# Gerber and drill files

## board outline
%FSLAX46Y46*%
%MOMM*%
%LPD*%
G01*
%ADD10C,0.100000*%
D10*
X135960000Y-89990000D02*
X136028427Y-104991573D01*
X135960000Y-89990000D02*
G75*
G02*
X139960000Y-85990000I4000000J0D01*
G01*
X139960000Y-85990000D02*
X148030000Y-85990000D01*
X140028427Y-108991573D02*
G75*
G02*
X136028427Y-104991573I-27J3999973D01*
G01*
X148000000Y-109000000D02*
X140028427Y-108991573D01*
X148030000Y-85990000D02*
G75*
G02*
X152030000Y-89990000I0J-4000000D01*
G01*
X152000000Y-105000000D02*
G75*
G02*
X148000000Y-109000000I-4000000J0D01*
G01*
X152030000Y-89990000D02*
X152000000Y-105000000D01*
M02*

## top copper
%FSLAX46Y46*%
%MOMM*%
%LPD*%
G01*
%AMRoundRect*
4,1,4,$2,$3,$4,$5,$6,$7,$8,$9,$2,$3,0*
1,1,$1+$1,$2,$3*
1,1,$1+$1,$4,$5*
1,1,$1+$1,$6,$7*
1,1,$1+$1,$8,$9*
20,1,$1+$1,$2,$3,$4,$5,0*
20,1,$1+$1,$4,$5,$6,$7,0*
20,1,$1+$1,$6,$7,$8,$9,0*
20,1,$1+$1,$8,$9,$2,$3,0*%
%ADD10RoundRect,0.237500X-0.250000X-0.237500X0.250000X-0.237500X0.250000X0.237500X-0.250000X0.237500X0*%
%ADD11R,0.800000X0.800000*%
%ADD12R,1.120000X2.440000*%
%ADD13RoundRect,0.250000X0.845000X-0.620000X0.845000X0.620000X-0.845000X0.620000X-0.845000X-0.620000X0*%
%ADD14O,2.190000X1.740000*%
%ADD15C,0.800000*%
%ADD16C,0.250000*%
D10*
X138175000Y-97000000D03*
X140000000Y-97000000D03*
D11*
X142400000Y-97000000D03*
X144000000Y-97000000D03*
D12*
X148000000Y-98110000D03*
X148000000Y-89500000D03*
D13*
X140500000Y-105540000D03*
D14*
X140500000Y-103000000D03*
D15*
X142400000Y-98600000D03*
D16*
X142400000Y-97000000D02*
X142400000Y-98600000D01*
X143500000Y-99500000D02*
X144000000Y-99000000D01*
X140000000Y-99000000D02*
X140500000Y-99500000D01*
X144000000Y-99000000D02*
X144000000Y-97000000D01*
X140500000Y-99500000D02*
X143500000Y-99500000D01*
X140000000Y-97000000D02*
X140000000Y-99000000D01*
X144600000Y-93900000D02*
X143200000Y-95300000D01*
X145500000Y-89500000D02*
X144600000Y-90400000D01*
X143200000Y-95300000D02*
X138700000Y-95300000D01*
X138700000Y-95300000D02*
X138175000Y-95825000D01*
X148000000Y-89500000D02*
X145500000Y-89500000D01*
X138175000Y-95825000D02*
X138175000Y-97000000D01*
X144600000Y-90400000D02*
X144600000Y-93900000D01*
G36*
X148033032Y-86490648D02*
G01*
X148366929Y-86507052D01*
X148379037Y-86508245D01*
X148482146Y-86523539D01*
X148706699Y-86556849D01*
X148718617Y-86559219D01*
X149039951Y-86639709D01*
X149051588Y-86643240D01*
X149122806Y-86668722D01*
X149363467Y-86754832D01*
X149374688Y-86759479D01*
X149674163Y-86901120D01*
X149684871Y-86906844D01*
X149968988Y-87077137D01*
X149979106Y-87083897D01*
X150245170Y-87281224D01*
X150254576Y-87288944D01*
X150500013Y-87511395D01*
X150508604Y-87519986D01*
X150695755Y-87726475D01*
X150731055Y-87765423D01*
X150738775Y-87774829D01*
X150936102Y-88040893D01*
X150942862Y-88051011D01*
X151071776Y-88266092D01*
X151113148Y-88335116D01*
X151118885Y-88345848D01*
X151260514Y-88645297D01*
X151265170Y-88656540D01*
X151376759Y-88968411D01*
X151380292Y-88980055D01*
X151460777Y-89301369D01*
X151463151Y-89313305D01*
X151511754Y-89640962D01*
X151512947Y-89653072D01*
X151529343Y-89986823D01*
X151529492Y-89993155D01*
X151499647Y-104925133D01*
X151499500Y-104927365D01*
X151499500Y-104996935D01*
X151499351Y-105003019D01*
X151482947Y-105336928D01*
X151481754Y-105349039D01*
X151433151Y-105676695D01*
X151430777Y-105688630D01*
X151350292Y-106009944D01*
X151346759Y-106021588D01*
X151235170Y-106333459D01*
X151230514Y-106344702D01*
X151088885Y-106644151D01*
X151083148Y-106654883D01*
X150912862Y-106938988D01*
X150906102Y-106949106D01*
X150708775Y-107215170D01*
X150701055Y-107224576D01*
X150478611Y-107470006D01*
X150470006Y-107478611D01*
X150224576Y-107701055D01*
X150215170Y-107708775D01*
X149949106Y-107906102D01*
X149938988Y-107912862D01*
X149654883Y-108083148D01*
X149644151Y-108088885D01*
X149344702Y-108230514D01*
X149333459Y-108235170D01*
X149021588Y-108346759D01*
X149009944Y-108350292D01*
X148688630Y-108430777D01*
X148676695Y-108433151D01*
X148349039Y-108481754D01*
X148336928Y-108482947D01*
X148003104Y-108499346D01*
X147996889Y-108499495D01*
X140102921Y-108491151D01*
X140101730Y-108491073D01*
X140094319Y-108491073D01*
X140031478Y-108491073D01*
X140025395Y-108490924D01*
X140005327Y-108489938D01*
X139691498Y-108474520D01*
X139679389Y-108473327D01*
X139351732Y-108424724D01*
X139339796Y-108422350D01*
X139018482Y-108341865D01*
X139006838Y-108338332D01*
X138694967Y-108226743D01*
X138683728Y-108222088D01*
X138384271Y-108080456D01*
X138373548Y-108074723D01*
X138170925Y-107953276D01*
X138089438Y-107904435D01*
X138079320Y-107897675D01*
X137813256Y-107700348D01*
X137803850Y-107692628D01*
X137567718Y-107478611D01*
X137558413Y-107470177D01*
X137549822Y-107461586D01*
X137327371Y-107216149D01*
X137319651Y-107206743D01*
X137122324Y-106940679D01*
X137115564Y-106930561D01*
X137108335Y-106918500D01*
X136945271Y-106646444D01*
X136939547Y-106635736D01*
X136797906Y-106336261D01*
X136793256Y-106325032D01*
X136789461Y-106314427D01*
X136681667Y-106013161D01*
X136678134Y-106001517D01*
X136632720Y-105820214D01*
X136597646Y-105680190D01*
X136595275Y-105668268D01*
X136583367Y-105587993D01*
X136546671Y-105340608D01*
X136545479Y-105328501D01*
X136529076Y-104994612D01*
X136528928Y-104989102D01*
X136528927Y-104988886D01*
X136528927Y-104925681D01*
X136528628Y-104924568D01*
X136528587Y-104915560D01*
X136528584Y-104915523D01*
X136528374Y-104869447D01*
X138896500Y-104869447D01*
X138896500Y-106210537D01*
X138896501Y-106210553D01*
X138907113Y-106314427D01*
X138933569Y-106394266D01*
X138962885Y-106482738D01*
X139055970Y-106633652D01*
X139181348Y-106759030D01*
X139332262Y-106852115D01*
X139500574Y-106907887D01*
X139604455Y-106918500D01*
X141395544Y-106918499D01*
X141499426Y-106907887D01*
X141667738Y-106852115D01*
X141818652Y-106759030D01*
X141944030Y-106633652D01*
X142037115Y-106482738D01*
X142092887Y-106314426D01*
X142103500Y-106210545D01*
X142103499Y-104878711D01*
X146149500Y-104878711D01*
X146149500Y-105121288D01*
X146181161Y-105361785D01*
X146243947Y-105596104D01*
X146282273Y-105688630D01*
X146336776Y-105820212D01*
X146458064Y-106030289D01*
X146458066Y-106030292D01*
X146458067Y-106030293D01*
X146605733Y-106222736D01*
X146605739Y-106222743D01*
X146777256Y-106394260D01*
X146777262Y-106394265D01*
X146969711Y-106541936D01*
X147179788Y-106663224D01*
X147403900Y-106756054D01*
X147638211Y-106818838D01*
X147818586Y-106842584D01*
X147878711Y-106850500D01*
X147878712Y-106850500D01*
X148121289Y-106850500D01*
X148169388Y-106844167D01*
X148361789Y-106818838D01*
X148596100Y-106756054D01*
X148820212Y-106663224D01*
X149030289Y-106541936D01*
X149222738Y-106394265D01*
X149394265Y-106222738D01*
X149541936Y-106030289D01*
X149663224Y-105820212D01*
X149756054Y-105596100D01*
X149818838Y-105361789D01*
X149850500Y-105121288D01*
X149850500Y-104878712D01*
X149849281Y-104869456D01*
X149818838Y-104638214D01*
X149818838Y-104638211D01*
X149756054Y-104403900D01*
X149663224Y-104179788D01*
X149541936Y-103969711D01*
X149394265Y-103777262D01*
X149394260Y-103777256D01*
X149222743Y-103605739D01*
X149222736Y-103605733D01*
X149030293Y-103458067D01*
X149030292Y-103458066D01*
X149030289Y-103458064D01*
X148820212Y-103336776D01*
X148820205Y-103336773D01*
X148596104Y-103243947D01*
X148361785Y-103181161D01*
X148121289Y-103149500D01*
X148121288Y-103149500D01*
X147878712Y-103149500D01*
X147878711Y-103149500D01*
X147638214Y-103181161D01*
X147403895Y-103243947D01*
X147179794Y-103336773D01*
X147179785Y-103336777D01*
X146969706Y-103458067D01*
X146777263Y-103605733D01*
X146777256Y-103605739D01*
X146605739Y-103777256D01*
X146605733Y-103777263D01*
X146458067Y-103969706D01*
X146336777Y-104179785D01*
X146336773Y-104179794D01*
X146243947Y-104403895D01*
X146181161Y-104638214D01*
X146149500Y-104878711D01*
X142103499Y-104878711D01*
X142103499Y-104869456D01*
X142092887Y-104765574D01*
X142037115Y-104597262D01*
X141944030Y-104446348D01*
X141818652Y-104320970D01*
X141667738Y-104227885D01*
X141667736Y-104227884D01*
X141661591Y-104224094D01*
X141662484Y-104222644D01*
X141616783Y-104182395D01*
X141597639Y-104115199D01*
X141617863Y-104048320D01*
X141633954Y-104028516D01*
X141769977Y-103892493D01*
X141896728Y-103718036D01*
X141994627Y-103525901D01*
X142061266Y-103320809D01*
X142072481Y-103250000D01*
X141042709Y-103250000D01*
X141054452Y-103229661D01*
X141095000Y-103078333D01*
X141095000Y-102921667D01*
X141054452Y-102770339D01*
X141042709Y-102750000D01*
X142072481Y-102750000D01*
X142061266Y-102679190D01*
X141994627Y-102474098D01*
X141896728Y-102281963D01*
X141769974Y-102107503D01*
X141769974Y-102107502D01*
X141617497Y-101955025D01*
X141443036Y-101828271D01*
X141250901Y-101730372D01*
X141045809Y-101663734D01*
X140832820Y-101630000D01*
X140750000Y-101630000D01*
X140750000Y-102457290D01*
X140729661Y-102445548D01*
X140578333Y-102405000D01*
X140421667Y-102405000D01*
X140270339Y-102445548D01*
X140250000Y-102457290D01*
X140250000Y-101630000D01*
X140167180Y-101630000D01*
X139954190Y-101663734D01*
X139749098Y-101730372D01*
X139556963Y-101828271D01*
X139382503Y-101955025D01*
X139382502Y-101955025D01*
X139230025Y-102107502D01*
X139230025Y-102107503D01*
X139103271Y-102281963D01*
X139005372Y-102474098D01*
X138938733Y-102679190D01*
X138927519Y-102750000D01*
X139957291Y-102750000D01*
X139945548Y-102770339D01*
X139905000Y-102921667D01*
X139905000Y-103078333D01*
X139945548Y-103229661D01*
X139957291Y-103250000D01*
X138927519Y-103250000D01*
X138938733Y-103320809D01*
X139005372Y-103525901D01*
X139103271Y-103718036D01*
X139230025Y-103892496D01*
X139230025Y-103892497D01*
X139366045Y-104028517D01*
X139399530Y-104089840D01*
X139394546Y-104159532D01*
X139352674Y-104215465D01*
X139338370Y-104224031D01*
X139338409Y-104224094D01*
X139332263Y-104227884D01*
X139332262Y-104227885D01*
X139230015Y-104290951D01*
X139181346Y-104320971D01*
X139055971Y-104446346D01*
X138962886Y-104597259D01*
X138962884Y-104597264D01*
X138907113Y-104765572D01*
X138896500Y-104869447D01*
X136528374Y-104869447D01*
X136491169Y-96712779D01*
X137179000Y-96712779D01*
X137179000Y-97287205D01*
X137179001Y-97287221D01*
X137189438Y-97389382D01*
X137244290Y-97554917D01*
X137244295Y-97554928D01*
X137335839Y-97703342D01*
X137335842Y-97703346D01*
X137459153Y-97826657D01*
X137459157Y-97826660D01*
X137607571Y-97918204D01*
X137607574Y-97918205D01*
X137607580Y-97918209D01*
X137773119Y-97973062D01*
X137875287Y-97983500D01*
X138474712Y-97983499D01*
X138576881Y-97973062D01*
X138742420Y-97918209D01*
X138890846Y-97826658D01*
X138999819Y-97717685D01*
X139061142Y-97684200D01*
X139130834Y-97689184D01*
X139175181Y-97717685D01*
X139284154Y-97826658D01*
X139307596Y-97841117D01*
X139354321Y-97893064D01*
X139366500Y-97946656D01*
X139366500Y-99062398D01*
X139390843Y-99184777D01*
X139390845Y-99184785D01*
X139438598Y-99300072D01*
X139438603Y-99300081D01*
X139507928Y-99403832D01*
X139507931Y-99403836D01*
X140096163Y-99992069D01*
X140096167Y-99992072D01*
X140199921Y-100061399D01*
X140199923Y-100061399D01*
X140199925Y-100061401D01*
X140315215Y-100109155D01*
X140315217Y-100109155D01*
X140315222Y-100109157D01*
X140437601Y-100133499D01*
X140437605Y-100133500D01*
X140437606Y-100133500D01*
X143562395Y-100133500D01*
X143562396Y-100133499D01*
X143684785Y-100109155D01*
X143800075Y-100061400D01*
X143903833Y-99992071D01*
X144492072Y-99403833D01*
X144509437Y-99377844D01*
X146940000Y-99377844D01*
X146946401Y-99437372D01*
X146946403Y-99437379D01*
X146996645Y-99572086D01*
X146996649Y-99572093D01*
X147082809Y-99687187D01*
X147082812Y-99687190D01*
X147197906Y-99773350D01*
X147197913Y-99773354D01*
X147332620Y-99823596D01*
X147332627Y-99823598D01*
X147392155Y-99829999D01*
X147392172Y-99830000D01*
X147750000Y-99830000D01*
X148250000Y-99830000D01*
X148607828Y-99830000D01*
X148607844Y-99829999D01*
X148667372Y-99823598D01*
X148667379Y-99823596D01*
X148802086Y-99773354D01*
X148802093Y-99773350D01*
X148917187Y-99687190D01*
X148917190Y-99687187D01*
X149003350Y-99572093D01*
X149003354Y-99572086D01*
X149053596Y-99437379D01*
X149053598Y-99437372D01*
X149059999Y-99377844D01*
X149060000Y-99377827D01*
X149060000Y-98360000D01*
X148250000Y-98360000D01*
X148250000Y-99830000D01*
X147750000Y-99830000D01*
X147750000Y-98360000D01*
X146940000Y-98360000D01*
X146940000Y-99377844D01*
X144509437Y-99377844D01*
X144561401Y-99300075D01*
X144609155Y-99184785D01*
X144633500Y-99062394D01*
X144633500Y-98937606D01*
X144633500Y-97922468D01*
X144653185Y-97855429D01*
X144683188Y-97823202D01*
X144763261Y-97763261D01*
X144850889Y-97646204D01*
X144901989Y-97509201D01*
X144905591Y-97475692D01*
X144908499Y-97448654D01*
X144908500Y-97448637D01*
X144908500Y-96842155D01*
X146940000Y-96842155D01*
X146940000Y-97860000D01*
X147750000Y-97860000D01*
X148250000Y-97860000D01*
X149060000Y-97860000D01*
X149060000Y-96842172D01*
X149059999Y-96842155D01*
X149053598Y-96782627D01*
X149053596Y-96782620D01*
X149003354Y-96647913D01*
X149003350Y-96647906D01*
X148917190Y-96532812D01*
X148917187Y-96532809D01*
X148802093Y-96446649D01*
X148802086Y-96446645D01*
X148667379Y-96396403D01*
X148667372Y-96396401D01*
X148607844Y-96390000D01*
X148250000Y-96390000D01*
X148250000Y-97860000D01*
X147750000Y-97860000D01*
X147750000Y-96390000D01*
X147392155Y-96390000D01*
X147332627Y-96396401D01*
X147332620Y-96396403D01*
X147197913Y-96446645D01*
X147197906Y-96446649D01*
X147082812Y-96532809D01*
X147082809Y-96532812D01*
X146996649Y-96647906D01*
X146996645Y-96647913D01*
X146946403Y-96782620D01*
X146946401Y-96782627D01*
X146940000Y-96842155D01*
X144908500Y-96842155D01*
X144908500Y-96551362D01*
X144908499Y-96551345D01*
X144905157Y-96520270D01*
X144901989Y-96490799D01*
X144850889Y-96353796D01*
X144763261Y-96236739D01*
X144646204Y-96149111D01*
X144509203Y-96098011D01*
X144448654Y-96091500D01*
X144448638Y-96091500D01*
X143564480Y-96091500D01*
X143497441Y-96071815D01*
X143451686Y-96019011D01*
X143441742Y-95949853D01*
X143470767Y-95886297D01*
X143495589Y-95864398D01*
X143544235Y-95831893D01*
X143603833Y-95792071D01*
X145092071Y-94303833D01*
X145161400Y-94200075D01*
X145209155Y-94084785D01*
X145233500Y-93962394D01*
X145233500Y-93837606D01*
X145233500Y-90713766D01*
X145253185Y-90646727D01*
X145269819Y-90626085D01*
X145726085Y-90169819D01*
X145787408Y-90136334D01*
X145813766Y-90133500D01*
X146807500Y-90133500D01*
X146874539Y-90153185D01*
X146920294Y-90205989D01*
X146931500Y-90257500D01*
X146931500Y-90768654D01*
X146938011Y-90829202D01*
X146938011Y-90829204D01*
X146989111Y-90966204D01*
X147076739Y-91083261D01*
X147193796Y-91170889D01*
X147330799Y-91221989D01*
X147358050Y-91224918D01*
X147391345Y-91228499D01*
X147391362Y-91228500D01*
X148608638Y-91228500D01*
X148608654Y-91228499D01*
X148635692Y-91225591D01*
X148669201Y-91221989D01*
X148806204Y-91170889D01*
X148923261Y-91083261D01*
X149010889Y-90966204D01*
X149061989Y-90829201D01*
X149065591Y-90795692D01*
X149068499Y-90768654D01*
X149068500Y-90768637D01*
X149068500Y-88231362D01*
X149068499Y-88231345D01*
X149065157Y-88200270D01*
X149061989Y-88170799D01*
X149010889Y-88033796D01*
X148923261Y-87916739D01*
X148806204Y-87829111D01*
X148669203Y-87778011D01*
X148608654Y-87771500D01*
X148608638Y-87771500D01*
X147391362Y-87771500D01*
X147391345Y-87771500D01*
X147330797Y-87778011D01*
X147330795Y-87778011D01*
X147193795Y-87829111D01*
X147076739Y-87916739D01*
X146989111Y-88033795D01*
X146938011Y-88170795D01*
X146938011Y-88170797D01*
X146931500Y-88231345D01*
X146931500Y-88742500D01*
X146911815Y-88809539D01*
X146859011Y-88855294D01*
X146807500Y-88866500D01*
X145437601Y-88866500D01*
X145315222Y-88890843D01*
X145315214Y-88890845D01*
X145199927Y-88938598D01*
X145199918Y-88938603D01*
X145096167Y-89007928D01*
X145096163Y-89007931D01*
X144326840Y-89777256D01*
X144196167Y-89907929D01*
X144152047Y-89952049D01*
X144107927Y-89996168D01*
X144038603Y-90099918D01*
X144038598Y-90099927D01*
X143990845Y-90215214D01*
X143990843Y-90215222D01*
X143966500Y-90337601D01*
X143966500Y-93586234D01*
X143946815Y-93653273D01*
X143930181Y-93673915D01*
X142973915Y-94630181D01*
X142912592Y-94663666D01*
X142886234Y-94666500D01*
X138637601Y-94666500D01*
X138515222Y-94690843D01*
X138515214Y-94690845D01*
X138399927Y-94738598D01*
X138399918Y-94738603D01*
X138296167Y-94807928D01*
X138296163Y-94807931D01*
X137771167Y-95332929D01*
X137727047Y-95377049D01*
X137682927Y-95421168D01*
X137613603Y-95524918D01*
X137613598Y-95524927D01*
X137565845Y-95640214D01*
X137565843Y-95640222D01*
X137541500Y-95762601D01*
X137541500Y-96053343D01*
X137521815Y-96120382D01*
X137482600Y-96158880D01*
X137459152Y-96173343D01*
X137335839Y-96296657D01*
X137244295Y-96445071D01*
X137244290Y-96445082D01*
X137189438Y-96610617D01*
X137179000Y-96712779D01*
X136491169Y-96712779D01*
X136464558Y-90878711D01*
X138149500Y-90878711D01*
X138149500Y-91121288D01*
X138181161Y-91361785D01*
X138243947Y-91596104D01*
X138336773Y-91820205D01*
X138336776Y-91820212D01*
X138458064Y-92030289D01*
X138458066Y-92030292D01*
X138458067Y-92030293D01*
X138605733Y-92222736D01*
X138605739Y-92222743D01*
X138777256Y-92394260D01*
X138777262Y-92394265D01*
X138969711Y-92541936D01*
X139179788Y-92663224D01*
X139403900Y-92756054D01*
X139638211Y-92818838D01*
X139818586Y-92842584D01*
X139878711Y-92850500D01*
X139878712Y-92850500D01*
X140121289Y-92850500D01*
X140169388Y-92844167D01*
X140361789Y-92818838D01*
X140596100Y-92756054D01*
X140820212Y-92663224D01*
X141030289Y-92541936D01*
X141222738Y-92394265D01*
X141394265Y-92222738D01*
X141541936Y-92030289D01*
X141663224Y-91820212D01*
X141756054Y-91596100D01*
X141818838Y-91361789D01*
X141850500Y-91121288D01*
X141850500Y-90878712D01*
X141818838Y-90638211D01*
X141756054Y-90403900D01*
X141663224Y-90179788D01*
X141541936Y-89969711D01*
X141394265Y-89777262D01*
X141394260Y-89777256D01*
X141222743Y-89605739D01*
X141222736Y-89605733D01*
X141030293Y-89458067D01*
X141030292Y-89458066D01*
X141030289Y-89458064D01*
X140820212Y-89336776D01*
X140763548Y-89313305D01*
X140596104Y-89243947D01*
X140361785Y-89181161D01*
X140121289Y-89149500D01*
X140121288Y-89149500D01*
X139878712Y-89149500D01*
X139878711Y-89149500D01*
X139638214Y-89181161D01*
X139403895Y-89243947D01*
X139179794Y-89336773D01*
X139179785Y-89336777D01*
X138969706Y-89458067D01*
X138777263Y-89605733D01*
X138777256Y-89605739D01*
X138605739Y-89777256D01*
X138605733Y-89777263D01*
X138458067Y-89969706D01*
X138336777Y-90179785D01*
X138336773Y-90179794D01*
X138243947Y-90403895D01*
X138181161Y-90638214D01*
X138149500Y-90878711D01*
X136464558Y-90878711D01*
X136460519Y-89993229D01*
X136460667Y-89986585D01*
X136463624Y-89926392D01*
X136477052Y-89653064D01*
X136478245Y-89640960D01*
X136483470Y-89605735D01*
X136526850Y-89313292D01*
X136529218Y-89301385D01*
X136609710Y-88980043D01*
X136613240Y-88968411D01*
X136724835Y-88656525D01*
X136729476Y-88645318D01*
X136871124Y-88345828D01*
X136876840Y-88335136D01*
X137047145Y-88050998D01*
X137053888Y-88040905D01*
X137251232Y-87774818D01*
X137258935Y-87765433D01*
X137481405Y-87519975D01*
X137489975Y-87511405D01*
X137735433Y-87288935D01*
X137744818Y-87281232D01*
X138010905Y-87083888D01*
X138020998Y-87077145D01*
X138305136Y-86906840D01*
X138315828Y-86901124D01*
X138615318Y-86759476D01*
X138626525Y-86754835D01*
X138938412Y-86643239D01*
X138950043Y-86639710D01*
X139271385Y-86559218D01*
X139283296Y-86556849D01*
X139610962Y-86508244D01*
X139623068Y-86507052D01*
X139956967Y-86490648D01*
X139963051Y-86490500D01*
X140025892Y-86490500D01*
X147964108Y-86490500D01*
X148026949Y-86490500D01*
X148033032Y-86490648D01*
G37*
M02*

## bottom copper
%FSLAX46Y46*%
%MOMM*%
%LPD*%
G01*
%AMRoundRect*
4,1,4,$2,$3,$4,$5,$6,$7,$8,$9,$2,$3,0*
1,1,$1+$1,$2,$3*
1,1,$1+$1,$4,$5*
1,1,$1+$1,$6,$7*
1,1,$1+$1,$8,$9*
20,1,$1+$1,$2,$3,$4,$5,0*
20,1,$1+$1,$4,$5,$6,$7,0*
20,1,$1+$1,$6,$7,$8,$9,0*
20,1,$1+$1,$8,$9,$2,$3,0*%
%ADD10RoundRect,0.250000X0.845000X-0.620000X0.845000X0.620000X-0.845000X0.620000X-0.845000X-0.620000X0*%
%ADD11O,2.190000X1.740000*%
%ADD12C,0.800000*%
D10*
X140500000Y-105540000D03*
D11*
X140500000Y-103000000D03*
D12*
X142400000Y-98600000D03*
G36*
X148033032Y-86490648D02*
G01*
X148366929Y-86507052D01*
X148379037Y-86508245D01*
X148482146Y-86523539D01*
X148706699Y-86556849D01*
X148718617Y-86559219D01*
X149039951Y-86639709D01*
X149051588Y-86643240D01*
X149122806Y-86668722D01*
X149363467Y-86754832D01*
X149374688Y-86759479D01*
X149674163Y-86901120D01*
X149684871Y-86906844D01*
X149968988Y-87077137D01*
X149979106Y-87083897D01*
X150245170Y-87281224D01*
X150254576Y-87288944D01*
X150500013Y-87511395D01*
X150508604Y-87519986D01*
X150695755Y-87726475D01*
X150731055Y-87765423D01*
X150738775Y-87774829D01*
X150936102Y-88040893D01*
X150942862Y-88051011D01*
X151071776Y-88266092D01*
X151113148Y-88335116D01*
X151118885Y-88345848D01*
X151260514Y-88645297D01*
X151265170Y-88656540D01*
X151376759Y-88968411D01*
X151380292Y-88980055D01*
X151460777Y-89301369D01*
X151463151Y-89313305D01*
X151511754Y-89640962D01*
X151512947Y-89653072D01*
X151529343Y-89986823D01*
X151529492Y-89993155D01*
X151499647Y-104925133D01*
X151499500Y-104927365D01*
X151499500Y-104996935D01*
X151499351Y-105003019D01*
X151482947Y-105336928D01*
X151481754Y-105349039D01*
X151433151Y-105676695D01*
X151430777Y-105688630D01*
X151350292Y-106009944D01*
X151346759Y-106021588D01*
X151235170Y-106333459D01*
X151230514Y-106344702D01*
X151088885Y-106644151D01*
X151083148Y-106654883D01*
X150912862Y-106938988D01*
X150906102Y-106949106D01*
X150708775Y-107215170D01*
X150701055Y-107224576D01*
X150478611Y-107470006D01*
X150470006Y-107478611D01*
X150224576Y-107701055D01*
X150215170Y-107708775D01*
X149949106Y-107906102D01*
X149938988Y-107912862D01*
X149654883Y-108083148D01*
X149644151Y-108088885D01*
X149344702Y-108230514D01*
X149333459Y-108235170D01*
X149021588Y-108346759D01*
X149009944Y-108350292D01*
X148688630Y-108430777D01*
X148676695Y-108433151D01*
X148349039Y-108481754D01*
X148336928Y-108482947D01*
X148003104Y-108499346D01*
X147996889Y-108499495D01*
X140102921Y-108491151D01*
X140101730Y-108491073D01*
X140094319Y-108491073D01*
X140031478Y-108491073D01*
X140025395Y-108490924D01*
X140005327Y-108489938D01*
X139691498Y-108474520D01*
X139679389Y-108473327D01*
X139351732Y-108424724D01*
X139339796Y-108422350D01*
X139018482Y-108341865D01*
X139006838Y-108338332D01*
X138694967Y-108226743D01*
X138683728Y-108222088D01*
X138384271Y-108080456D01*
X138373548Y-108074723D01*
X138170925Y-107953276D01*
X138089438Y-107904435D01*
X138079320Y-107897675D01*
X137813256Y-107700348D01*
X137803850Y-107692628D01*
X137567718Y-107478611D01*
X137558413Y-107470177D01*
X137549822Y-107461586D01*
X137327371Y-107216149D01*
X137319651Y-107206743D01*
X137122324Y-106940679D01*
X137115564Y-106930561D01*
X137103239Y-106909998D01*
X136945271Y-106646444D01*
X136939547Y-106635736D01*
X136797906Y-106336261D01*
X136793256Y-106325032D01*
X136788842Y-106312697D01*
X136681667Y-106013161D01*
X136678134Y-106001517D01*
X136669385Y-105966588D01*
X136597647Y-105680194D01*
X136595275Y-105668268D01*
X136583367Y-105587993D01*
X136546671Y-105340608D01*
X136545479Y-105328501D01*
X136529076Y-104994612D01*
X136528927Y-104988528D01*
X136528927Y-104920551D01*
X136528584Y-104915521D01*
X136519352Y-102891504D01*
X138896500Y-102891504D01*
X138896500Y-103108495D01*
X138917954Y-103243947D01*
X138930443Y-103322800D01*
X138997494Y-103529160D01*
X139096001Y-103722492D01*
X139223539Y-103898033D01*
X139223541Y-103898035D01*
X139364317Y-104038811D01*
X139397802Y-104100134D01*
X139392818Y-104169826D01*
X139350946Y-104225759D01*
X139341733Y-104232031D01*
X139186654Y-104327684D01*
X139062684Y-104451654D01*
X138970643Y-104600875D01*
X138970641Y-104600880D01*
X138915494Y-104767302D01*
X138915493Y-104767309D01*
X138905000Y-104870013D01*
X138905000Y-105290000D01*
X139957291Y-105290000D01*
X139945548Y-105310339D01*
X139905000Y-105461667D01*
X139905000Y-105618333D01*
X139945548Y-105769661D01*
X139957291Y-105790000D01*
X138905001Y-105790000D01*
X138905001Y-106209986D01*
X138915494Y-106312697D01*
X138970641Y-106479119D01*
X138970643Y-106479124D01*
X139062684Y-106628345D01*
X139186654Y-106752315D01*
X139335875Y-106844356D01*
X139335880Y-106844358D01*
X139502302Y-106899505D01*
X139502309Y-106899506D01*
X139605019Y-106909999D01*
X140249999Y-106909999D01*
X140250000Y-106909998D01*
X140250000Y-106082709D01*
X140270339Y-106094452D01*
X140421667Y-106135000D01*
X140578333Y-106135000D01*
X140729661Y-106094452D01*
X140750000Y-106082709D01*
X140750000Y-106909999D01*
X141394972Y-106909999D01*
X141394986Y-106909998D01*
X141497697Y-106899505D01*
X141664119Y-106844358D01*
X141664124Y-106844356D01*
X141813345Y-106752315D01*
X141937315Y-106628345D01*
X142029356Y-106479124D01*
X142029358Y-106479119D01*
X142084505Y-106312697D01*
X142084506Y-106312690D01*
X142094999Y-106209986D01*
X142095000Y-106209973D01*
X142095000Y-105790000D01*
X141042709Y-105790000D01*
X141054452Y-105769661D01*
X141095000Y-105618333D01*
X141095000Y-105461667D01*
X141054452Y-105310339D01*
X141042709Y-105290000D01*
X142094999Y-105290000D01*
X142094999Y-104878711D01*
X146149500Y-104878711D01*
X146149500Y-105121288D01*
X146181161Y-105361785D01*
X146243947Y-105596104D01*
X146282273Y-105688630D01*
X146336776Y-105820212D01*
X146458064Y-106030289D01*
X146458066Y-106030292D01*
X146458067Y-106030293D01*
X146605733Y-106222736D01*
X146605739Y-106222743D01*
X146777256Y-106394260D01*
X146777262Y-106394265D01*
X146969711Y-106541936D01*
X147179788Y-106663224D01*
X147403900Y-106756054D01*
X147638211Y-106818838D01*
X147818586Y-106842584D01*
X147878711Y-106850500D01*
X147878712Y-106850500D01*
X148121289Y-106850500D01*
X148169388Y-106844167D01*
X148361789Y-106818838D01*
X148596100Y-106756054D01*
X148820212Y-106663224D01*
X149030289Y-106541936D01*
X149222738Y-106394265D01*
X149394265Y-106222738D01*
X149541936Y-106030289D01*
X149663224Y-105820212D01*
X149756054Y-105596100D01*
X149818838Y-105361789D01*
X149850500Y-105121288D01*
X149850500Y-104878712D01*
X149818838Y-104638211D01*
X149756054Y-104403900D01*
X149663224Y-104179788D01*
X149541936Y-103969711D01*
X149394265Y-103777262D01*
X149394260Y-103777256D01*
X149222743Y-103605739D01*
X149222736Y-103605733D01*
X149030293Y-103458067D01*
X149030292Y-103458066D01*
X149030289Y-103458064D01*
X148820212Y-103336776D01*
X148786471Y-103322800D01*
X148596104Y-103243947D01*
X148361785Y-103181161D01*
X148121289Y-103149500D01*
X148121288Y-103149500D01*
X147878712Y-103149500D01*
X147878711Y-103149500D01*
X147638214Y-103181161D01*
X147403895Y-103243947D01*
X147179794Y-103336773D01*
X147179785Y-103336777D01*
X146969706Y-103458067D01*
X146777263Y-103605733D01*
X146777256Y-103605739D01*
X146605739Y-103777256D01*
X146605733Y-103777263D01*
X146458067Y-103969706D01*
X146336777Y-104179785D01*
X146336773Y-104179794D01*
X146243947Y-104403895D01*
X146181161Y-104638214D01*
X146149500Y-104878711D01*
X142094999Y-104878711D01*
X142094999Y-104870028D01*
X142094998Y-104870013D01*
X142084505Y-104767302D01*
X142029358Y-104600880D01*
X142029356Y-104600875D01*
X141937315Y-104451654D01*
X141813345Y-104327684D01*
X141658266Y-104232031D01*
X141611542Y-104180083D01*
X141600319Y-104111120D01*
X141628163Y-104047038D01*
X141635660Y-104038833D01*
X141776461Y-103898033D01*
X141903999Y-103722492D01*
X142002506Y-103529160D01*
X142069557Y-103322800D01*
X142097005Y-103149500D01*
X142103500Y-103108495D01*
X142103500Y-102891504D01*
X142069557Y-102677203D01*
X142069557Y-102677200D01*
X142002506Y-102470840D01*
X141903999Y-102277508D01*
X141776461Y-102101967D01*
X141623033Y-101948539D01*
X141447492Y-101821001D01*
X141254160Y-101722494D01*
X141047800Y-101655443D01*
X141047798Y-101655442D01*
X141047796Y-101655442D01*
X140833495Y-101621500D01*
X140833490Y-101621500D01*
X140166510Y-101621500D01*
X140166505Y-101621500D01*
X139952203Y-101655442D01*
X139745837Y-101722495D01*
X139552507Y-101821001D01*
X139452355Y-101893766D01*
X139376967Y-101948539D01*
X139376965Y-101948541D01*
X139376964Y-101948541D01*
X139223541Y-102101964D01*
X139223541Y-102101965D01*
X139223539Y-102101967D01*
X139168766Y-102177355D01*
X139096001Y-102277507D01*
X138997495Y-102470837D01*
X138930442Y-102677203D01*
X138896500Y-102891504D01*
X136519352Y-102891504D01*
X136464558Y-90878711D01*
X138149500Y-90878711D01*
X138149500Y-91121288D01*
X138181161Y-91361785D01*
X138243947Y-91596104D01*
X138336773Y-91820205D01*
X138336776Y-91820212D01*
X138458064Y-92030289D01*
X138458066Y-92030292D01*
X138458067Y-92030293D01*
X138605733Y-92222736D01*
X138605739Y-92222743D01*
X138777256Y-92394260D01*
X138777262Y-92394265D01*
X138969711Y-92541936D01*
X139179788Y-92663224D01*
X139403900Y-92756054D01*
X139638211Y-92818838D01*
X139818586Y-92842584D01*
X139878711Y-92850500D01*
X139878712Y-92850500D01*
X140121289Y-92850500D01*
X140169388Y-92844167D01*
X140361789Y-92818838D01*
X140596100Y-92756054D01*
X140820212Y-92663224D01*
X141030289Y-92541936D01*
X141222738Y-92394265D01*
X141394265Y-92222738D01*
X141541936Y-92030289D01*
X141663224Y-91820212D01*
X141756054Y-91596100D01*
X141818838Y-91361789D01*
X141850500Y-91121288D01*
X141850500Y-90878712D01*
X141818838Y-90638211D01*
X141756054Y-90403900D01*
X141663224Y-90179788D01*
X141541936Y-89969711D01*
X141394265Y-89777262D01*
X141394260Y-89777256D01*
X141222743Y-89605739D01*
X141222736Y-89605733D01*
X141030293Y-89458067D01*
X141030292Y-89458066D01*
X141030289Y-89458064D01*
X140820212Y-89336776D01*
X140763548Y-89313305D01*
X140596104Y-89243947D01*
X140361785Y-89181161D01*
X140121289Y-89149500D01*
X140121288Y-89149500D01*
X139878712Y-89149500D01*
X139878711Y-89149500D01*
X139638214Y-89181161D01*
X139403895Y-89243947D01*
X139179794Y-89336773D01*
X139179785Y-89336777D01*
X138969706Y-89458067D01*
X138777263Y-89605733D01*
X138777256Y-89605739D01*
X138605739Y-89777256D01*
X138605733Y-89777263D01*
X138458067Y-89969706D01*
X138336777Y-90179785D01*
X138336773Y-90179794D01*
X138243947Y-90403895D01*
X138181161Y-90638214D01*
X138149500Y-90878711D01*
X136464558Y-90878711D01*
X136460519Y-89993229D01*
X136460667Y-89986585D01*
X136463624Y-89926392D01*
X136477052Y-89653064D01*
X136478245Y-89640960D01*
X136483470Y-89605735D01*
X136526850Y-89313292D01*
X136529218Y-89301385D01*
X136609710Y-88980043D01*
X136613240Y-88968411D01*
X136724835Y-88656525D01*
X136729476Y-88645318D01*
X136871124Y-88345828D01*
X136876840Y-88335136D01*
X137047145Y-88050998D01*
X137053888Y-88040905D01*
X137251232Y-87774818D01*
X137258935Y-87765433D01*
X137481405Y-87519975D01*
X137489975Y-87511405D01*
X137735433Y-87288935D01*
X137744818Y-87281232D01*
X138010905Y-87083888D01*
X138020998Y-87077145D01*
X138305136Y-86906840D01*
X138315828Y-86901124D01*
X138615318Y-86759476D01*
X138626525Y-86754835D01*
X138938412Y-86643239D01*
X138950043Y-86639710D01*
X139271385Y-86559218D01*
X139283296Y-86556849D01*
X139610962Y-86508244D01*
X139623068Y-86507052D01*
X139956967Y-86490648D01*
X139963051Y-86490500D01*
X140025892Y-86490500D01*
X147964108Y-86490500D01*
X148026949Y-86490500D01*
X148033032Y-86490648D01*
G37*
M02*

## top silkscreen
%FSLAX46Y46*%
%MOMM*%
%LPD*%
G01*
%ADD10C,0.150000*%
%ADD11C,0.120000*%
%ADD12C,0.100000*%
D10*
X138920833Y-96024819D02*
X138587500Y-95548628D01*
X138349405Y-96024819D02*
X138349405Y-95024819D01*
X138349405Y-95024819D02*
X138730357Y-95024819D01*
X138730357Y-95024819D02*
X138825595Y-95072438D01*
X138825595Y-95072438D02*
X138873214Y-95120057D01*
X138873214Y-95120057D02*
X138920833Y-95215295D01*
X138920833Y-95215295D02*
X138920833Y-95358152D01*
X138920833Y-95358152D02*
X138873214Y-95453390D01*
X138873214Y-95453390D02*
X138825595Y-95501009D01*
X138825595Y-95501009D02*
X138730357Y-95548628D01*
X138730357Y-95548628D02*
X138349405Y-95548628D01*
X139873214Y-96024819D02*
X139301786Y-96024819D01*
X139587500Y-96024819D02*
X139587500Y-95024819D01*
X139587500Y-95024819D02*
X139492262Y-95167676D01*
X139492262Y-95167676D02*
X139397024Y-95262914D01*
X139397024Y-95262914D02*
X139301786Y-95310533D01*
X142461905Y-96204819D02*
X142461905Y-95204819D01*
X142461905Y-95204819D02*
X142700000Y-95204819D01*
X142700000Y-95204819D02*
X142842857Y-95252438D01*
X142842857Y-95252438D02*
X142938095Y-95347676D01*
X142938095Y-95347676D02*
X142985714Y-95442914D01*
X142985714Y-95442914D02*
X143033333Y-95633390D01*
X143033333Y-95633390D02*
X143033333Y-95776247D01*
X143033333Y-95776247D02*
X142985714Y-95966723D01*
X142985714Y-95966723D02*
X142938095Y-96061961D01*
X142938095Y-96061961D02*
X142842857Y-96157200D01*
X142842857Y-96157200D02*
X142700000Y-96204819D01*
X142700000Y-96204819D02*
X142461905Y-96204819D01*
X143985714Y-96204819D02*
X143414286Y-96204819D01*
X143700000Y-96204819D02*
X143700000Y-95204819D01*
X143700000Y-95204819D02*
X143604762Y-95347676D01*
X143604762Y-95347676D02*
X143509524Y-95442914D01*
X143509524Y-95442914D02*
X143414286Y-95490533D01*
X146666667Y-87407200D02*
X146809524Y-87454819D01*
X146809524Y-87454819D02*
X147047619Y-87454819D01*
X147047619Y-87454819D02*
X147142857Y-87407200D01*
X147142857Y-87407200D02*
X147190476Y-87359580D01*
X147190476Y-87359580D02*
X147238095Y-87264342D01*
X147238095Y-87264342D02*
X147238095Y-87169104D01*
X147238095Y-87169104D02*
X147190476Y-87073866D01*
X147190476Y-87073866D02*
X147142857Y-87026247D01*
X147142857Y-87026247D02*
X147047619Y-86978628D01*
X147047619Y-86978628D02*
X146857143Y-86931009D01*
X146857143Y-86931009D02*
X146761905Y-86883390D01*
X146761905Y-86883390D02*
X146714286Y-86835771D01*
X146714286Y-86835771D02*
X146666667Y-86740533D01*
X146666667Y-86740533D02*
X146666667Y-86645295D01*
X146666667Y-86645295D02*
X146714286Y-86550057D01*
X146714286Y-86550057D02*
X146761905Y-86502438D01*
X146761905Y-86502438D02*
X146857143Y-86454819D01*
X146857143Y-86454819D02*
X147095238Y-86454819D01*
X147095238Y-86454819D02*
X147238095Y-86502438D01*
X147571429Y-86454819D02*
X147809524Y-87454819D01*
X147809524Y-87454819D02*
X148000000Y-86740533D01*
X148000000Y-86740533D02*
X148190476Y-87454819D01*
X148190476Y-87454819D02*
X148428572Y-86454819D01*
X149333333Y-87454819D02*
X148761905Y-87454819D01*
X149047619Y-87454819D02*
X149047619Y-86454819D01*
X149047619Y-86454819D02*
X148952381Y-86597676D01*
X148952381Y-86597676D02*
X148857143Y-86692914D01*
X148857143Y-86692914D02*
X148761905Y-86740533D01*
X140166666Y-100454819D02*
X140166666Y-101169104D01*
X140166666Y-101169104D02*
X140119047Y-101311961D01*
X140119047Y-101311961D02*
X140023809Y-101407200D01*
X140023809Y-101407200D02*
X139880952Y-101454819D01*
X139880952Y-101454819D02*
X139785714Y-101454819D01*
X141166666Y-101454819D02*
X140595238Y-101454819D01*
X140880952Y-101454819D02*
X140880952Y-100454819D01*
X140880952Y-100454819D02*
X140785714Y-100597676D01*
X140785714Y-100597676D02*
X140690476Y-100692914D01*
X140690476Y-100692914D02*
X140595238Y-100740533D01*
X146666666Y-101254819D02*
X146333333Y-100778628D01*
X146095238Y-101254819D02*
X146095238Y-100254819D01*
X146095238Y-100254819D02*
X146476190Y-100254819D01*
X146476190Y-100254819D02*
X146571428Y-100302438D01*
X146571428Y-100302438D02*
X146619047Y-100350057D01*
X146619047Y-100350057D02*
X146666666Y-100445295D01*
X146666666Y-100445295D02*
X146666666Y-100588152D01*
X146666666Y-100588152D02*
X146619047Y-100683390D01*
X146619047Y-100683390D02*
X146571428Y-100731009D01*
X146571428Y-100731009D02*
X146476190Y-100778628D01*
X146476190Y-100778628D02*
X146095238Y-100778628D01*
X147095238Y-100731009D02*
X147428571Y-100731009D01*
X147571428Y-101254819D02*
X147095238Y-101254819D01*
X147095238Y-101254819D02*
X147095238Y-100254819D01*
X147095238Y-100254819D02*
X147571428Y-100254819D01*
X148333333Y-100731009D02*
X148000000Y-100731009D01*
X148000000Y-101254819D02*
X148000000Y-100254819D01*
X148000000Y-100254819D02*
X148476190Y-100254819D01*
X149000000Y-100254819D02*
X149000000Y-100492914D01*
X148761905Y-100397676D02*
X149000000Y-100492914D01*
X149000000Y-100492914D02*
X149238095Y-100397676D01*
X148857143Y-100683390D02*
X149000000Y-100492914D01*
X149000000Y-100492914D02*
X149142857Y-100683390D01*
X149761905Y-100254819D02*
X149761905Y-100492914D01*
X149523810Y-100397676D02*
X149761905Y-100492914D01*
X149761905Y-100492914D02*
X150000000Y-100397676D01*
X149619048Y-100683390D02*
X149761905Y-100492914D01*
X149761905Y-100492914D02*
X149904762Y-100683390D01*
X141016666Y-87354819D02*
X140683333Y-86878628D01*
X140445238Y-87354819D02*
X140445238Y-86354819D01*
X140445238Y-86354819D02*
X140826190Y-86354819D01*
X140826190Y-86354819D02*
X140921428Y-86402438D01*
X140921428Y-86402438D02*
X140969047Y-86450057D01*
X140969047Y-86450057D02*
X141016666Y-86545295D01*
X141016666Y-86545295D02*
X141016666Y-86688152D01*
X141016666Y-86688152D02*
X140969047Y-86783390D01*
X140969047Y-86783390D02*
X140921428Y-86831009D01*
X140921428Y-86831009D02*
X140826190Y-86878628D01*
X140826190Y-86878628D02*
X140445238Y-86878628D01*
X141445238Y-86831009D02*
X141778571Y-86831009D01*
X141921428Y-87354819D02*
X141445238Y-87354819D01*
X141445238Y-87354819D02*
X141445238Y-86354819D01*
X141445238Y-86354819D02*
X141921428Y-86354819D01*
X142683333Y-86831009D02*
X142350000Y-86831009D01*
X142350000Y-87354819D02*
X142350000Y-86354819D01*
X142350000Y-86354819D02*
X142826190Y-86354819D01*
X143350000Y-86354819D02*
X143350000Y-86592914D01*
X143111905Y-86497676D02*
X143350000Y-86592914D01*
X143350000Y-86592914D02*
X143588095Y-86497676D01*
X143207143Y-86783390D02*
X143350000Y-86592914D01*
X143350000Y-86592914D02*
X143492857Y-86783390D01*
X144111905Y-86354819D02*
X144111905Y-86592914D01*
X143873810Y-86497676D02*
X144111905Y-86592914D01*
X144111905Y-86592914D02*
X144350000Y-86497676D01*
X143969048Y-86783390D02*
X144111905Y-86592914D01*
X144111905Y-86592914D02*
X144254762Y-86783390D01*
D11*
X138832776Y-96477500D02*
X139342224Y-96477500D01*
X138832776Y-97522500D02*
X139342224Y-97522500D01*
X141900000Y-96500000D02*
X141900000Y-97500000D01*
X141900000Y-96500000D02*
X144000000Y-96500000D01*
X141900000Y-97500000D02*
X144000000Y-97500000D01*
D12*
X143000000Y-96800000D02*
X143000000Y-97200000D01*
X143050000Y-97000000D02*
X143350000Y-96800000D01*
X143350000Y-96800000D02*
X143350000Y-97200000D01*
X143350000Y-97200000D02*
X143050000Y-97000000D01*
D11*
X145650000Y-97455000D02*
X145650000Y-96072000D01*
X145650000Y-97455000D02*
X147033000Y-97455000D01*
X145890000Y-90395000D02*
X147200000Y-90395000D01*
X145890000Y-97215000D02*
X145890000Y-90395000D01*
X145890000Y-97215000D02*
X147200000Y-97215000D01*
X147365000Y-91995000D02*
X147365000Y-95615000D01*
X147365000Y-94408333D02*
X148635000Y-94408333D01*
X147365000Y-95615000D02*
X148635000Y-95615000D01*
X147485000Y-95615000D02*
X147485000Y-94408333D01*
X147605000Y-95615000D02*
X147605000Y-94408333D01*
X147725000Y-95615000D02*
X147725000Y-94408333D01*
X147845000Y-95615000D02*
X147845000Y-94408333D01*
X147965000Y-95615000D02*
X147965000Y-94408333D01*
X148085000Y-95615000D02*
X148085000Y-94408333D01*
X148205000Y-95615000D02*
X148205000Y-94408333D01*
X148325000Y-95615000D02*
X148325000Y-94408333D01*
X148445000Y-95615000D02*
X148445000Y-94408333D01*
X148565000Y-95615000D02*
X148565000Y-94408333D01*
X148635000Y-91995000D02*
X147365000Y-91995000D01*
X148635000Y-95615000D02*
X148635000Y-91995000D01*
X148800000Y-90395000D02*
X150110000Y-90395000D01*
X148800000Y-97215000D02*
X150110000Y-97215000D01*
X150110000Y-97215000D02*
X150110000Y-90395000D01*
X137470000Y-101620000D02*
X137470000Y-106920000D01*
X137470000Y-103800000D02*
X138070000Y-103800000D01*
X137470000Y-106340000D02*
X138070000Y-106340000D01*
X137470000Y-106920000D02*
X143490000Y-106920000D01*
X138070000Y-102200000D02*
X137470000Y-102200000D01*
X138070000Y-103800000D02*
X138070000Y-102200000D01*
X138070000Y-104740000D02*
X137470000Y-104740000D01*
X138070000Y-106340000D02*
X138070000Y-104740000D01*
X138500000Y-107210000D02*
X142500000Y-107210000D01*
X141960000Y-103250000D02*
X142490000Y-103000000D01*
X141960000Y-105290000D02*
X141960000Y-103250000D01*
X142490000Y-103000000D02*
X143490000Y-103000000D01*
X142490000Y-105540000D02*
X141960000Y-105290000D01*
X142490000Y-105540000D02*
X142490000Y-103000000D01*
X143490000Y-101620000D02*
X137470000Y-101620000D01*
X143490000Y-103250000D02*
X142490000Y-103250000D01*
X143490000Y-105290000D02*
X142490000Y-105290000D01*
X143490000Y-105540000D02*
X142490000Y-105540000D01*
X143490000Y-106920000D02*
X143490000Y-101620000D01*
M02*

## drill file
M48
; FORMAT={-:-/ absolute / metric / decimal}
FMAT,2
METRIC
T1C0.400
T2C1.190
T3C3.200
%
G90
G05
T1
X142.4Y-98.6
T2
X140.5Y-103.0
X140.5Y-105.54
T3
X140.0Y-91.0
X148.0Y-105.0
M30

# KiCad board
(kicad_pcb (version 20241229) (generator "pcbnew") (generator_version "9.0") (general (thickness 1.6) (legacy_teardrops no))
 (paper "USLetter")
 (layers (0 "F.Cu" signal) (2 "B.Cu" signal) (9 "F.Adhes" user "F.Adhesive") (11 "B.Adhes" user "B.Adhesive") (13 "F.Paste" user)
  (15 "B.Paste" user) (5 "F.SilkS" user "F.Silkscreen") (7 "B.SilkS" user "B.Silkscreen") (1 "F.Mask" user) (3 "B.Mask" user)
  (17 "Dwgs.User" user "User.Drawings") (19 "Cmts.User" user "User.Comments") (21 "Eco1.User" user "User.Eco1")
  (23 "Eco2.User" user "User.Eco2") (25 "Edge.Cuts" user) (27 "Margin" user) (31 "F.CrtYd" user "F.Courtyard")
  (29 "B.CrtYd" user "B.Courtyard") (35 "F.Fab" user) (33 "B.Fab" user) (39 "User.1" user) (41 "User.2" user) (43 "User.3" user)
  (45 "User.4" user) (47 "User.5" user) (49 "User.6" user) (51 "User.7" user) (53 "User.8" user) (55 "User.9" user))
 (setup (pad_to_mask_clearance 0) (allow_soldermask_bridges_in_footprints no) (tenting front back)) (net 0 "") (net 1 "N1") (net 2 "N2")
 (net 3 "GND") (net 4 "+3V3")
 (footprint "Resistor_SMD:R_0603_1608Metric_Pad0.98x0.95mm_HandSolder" (layer "F.Cu") (at 139.0875 97)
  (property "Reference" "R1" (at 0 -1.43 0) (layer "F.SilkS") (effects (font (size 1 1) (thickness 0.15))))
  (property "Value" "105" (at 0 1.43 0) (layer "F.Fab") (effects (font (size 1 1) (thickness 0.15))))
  (fp_line (start -0.254724 -0.5225) (end 0.254724 -0.5225) (stroke (width 0.12) (type solid)) (layer "F.SilkS"))
  (fp_line (start -0.254724 0.5225) (end 0.254724 0.5225) (stroke (width 0.12) (type solid)) (layer "F.SilkS"))
  (pad "1" smd roundrect (at -0.9125 0) (size 0.975 0.95) (layers "F.Cu" "F.Mask" "F.Paste") (roundrect_rratio 0.25) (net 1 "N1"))
  (pad "2" smd roundrect (at 0.9125 0) (size 0.975 0.95) (layers "F.Cu" "F.Mask" "F.Paste") (roundrect_rratio 0.25) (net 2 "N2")))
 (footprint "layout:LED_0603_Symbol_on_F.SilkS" (layer "F.Cu") (at 143.2 97)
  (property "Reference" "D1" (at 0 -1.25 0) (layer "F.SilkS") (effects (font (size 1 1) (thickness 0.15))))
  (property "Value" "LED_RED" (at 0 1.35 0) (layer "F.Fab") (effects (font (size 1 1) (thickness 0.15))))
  (fp_line (start -1.3 -0.5) (end -1.3 0.5) (stroke (width 0.12) (type solid)) (layer "F.SilkS"))
  (fp_line (start -1.3 -0.5) (end 0.8 -0.5) (stroke (width 0.12) (type solid)) (layer "F.SilkS"))
  (fp_line (start -1.3 0.5) (end 0.8 0.5) (stroke (width 0.12) (type solid)) (layer "F.SilkS"))
  (fp_line (start -0.2 -0.2) (end -0.2 0.2) (stroke (width 0.1) (type solid)) (layer "F.SilkS"))
  (fp_line (start -0.15 0) (end 0.15 -0.2) (stroke (width 0.1) (type solid)) (layer "F.SilkS"))
  (fp_line (start 0.15 -0.2) (end 0.15 0.2) (stroke (width 0.1) (type solid)) (layer "F.SilkS"))
  (fp_line (start 0.15 0.2) (end -0.15 0) (stroke (width 0.1) (type solid)) (layer "F.SilkS"))
  (pad "1" smd rect (at -0.8 0 180) (size 0.8 0.8) (layers "F.Cu" "F.Mask" "F.Paste") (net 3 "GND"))
  (pad "2" smd rect (at 0.8 0 180) (size 0.8 0.8) (layers "F.Cu" "F.Mask" "F.Paste") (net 2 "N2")))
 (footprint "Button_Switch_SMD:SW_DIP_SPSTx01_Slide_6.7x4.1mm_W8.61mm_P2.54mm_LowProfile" (layer "F.Cu") (at 148 93.805 90)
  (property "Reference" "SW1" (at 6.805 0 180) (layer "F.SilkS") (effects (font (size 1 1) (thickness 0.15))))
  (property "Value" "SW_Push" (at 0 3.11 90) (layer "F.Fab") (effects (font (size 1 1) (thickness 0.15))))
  (fp_line (start -3.65 -2.35) (end -2.267 -2.35) (stroke (width 0.12) (type solid)) (layer "F.SilkS"))
  (fp_line (start -3.65 -2.35) (end -3.65 -0.967) (stroke (width 0.12) (type solid)) (layer "F.SilkS"))
  (fp_line (start 3.41 -2.11) (end 3.41 -0.8) (stroke (width 0.12) (type solid)) (layer "F.SilkS"))
  (fp_line (start -3.41 -2.11) (end 3.41 -2.11) (stroke (width 0.12) (type solid)) (layer "F.SilkS"))
  (fp_line (start -3.41 -2.11) (end -3.41 -0.8) (stroke (width 0.12) (type solid)) (layer "F.SilkS"))
  (fp_line (start 1.81 -0.635) (end -1.81 -0.635) (stroke (width 0.12) (type solid)) (layer "F.SilkS"))
  (fp_line (start -0.603333 -0.635) (end -0.603333 0.635) (stroke (width 0.12) (type solid)) (layer "F.SilkS"))
  (fp_line (start -1.81 -0.635) (end -1.81 0.635) (stroke (width 0.12) (type solid)) (layer "F.SilkS"))
  (fp_line (start -1.81 -0.515) (end -0.603333 -0.515) (stroke (width 0.12) (type solid)) (layer "F.SilkS"))
  (fp_line (start -1.81 -0.395) (end -0.603333 -0.395) (stroke (width 0.12) (type solid)) (layer "F.SilkS"))
  (fp_line (start -1.81 -0.275) (end -0.603333 -0.275) (stroke (width 0.12) (type solid)) (layer "F.SilkS"))
  (fp_line (start -1.81 -0.155) (end -0.603333 -0.155) (stroke (width 0.12) (type solid)) (layer "F.SilkS"))
  (fp_line (start -1.81 -0.035) (end -0.603333 -0.035) (stroke (width 0.12) (type solid)) (layer "F.SilkS"))
  (fp_line (start -1.81 0.085) (end -0.603333 0.085) (stroke (width 0.12) (type solid)) (layer "F.SilkS"))
  (fp_line (start -1.81 0.205) (end -0.603333 0.205) (stroke (width 0.12) (type solid)) (layer "F.SilkS"))
  (fp_line (start -1.81 0.325) (end -0.603333 0.325) (stroke (width 0.12) (type solid)) (layer "F.SilkS"))
  (fp_line (start -1.81 0.445) (end -0.603333 0.445) (stroke (width 0.12) (type solid)) (layer "F.SilkS"))
  (fp_line (start -1.81 0.565) (end -0.603333 0.565) (stroke (width 0.12) (type solid)) (layer "F.SilkS"))
  (fp_line (start 1.81 0.635) (end 1.81 -0.635) (stroke (width 0.12) (type solid)) (layer "F.SilkS"))
  (fp_line (start -1.81 0.635) (end 1.81 0.635) (stroke (width 0.12) (type solid)) (layer "F.SilkS"))
  (fp_line (start 3.41 0.8) (end 3.41 2.11) (stroke (width 0.12) (type solid)) (layer "F.SilkS"))
  (fp_line (start -3.41 0.8) (end -3.41 2.11) (stroke (width 0.12) (type solid)) (layer "F.SilkS"))
  (fp_line (start -3.41 2.11) (end 3.41 2.11) (stroke (width 0.12) (type solid)) (layer "F.SilkS"))
  (pad "1" smd rect (at -4.305 0 90) (size 2.44 1.12) (layers "F.Cu" "F.Mask" "F.Paste") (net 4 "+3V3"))
  (pad "2" smd rect (at 4.305 0 90) (size 2.44 1.12) (layers "F.Cu" "F.Mask" "F.Paste") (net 1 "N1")))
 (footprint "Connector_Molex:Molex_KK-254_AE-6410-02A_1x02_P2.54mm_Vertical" (layer "F.Cu") (at 140.5 105.54 90)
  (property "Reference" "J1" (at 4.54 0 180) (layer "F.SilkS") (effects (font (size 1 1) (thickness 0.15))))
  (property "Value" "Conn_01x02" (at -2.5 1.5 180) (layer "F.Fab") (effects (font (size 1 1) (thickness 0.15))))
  (fp_line (start 3.92 -3.03) (end -1.38 -3.03) (stroke (width 0.12) (type solid)) (layer "F.SilkS"))
  (fp_line (start 1.74 -3.03) (end 1.74 -2.43) (stroke (width 0.12) (type solid)) (layer "F.SilkS"))
  (fp_line (start -0.8 -3.03) (end -0.8 -2.43) (stroke (width 0.12) (type solid)) (layer "F.SilkS"))
  (fp_line (start -1.38 -3.03) (end -1.38 2.99) (stroke (width 0.12) (type solid)) (layer "F.SilkS"))
  (fp_line (start 3.34 -2.43) (end 3.34 -3.03) (stroke (width 0.12) (type solid)) (layer "F.SilkS"))
  (fp_line (start 1.74 -2.43) (end 3.34 -2.43) (stroke (width 0.12) (type solid)) (layer "F.SilkS"))
  (fp_line (start 0.8 -2.43) (end 0.8 -3.03) (stroke (width 0.12) (type solid)) (layer "F.SilkS"))
  (fp_line (start -0.8 -2.43) (end 0.8 -2.43) (stroke (width 0.12) (type solid)) (layer "F.SilkS"))
  (fp_line (start -1.67 -2) (end -1.67 2) (stroke (width 0.12) (type solid)) (layer "F.SilkS"))
  (fp_line (start 2.29 1.46) (end 2.54 1.99) (stroke (width 0.12) (type solid)) (layer "F.SilkS"))
  (fp_line (start 0.25 1.46) (end 2.29 1.46) (stroke (width 0.12) (type solid)) (layer "F.SilkS"))
  (fp_line (start 2.54 1.99) (end 2.54 2.99) (stroke (width 0.12) (type solid)) (layer "F.SilkS"))
  (fp_line (start 0 1.99) (end 0.25 1.46) (stroke (width 0.12) (type solid)) (layer "F.SilkS"))
  (fp_line (start 0 1.99) (end 2.54 1.99) (stroke (width 0.12) (type solid)) (layer "F.SilkS"))
  (fp_line (start 3.92 2.99) (end 3.92 -3.03) (stroke (width 0.12) (type solid)) (layer "F.SilkS"))
  (fp_line (start 2.29 2.99) (end 2.29 1.99) (stroke (width 0.12) (type solid)) (layer "F.SilkS"))
  (fp_line (start 0.25 2.99) (end 0.25 1.99) (stroke (width 0.12) (type solid)) (layer "F.SilkS"))
  (fp_line (start 0 2.99) (end 0 1.99) (stroke (width 0.12) (type solid)) (layer "F.SilkS"))
  (fp_line (start -1.38 2.99) (end 3.92 2.99) (stroke (width 0.12) (type solid)) (layer "F.SilkS"))
  (pad "1" thru_hole roundrect (at 0 0 90) (size 1.74 2.19) (drill 1.19) (layers "*.Cu" "*.Mask") (remove_unused_layers no)
   (roundrect_rratio 0.143678) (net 3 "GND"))
  (pad "2" thru_hole oval (at 2.54 0 90) (size 1.74 2.19) (drill 1.19) (layers "*.Cu" "*.Mask") (remove_unused_layers no) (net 4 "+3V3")))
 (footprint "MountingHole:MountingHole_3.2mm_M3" (layer "F.Cu") (at 148 105)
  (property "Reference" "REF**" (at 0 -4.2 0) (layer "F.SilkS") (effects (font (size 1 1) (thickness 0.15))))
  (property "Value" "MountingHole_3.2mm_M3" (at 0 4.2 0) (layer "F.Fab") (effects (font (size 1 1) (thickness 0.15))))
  (pad "" np_thru_hole circle (at 0 0) (size 3.2 3.2) (drill 3.2) (layers "*.Cu" "*.Mask")))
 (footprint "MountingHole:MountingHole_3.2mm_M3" (layer "F.Cu") (at 140 91)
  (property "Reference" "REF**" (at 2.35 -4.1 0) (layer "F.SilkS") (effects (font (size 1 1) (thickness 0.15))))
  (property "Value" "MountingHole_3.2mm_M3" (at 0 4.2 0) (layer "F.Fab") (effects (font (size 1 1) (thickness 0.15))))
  (pad "" np_thru_hole circle (at 0 0) (size 3.2 3.2) (drill 3.2) (layers "*.Cu" "*.Mask")))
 (gr_line (start 135.96 89.99) (end 136.028427 104.991573) (stroke (width 0.1) (type default)) (layer "Edge.Cuts"))
 (gr_arc (start 135.96 89.99) (mid 137.131573 87.161573) (end 139.96 85.99) (stroke (width 0.1) (type default)) (layer "Edge.Cuts"))
 (gr_line (start 139.96 85.99) (end 148.03 85.99) (stroke (width 0.1) (type default)) (layer "Edge.Cuts"))
 (gr_arc (start 140.028427 108.991573) (mid 137.2 107.82) (end 136.028427 104.991573) (stroke (width 0.1) (type default))
  (layer "Edge.Cuts"))
 (gr_line (start 148 109) (end 140.028427 108.991573) (stroke (width 0.1) (type default)) (layer "Edge.Cuts"))
 (gr_arc (start 148.03 85.99) (mid 150.858427 87.161573) (end 152.03 89.99) (stroke (width 0.1) (type default)) (layer "Edge.Cuts"))
 (gr_arc (start 152 105) (mid 150.828427 107.828427) (end 148 109) (stroke (width 0.1) (type default)) (layer "Edge.Cuts"))
 (gr_line (start 152.03 89.99) (end 152 105) (stroke (width 0.1) (type default)) (layer "Edge.Cuts"))
 (segment (start 142.4 97) (end 142.4 98.6) (width 0.25) (layer "F.Cu") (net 3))
 (via (at 142.4 98.6) (size 0.8) (drill 0.4) (layers "F.Cu" "B.Cu") (free yes) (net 3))
 (segment (start 143.5 99.5) (end 144 99) (width 0.25) (layer "F.Cu") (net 2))
 (segment (start 140 99) (end 140.5 99.5) (width 0.25) (layer "F.Cu") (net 2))
 (segment (start 144 99) (end 144 97) (width 0.25) (layer "F.Cu") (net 2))
 (segment (start 140.5 99.5) (end 143.5 99.5) (width 0.25) (layer "F.Cu") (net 2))
 (segment (start 140 97) (end 140 99) (width 0.25) (layer "F.Cu") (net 2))
 (segment (start 144.6 93.9) (end 143.2 95.3) (width 0.25) (layer "F.Cu") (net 1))
 (segment (start 145.5 89.5) (end 144.6 90.4) (width 0.25) (layer "F.Cu") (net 1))
 (segment (start 143.2 95.3) (end 138.7 95.3) (width 0.25) (layer "F.Cu") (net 1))
 (segment (start 138.7 95.3) (end 138.175 95.825) (width 0.25) (layer "F.Cu") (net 1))
 (segment (start 148 89.5) (end 145.5 89.5) (width 0.25) (layer "F.Cu") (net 1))
 (segment (start 138.175 95.825) (end 138.175 97) (width 0.25) (layer "F.Cu") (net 1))
 (segment (start 144.6 90.4) (end 144.6 93.9) (width 0.25) (layer "F.Cu") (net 1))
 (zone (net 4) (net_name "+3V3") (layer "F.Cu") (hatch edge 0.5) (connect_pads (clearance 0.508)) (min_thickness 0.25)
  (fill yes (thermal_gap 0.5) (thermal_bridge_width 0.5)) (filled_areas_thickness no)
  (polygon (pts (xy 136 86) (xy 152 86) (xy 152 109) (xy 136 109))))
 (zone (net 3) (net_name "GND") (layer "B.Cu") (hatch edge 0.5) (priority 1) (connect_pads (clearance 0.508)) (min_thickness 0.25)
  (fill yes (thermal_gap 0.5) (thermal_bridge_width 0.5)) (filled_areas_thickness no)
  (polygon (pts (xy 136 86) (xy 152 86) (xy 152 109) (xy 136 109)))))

